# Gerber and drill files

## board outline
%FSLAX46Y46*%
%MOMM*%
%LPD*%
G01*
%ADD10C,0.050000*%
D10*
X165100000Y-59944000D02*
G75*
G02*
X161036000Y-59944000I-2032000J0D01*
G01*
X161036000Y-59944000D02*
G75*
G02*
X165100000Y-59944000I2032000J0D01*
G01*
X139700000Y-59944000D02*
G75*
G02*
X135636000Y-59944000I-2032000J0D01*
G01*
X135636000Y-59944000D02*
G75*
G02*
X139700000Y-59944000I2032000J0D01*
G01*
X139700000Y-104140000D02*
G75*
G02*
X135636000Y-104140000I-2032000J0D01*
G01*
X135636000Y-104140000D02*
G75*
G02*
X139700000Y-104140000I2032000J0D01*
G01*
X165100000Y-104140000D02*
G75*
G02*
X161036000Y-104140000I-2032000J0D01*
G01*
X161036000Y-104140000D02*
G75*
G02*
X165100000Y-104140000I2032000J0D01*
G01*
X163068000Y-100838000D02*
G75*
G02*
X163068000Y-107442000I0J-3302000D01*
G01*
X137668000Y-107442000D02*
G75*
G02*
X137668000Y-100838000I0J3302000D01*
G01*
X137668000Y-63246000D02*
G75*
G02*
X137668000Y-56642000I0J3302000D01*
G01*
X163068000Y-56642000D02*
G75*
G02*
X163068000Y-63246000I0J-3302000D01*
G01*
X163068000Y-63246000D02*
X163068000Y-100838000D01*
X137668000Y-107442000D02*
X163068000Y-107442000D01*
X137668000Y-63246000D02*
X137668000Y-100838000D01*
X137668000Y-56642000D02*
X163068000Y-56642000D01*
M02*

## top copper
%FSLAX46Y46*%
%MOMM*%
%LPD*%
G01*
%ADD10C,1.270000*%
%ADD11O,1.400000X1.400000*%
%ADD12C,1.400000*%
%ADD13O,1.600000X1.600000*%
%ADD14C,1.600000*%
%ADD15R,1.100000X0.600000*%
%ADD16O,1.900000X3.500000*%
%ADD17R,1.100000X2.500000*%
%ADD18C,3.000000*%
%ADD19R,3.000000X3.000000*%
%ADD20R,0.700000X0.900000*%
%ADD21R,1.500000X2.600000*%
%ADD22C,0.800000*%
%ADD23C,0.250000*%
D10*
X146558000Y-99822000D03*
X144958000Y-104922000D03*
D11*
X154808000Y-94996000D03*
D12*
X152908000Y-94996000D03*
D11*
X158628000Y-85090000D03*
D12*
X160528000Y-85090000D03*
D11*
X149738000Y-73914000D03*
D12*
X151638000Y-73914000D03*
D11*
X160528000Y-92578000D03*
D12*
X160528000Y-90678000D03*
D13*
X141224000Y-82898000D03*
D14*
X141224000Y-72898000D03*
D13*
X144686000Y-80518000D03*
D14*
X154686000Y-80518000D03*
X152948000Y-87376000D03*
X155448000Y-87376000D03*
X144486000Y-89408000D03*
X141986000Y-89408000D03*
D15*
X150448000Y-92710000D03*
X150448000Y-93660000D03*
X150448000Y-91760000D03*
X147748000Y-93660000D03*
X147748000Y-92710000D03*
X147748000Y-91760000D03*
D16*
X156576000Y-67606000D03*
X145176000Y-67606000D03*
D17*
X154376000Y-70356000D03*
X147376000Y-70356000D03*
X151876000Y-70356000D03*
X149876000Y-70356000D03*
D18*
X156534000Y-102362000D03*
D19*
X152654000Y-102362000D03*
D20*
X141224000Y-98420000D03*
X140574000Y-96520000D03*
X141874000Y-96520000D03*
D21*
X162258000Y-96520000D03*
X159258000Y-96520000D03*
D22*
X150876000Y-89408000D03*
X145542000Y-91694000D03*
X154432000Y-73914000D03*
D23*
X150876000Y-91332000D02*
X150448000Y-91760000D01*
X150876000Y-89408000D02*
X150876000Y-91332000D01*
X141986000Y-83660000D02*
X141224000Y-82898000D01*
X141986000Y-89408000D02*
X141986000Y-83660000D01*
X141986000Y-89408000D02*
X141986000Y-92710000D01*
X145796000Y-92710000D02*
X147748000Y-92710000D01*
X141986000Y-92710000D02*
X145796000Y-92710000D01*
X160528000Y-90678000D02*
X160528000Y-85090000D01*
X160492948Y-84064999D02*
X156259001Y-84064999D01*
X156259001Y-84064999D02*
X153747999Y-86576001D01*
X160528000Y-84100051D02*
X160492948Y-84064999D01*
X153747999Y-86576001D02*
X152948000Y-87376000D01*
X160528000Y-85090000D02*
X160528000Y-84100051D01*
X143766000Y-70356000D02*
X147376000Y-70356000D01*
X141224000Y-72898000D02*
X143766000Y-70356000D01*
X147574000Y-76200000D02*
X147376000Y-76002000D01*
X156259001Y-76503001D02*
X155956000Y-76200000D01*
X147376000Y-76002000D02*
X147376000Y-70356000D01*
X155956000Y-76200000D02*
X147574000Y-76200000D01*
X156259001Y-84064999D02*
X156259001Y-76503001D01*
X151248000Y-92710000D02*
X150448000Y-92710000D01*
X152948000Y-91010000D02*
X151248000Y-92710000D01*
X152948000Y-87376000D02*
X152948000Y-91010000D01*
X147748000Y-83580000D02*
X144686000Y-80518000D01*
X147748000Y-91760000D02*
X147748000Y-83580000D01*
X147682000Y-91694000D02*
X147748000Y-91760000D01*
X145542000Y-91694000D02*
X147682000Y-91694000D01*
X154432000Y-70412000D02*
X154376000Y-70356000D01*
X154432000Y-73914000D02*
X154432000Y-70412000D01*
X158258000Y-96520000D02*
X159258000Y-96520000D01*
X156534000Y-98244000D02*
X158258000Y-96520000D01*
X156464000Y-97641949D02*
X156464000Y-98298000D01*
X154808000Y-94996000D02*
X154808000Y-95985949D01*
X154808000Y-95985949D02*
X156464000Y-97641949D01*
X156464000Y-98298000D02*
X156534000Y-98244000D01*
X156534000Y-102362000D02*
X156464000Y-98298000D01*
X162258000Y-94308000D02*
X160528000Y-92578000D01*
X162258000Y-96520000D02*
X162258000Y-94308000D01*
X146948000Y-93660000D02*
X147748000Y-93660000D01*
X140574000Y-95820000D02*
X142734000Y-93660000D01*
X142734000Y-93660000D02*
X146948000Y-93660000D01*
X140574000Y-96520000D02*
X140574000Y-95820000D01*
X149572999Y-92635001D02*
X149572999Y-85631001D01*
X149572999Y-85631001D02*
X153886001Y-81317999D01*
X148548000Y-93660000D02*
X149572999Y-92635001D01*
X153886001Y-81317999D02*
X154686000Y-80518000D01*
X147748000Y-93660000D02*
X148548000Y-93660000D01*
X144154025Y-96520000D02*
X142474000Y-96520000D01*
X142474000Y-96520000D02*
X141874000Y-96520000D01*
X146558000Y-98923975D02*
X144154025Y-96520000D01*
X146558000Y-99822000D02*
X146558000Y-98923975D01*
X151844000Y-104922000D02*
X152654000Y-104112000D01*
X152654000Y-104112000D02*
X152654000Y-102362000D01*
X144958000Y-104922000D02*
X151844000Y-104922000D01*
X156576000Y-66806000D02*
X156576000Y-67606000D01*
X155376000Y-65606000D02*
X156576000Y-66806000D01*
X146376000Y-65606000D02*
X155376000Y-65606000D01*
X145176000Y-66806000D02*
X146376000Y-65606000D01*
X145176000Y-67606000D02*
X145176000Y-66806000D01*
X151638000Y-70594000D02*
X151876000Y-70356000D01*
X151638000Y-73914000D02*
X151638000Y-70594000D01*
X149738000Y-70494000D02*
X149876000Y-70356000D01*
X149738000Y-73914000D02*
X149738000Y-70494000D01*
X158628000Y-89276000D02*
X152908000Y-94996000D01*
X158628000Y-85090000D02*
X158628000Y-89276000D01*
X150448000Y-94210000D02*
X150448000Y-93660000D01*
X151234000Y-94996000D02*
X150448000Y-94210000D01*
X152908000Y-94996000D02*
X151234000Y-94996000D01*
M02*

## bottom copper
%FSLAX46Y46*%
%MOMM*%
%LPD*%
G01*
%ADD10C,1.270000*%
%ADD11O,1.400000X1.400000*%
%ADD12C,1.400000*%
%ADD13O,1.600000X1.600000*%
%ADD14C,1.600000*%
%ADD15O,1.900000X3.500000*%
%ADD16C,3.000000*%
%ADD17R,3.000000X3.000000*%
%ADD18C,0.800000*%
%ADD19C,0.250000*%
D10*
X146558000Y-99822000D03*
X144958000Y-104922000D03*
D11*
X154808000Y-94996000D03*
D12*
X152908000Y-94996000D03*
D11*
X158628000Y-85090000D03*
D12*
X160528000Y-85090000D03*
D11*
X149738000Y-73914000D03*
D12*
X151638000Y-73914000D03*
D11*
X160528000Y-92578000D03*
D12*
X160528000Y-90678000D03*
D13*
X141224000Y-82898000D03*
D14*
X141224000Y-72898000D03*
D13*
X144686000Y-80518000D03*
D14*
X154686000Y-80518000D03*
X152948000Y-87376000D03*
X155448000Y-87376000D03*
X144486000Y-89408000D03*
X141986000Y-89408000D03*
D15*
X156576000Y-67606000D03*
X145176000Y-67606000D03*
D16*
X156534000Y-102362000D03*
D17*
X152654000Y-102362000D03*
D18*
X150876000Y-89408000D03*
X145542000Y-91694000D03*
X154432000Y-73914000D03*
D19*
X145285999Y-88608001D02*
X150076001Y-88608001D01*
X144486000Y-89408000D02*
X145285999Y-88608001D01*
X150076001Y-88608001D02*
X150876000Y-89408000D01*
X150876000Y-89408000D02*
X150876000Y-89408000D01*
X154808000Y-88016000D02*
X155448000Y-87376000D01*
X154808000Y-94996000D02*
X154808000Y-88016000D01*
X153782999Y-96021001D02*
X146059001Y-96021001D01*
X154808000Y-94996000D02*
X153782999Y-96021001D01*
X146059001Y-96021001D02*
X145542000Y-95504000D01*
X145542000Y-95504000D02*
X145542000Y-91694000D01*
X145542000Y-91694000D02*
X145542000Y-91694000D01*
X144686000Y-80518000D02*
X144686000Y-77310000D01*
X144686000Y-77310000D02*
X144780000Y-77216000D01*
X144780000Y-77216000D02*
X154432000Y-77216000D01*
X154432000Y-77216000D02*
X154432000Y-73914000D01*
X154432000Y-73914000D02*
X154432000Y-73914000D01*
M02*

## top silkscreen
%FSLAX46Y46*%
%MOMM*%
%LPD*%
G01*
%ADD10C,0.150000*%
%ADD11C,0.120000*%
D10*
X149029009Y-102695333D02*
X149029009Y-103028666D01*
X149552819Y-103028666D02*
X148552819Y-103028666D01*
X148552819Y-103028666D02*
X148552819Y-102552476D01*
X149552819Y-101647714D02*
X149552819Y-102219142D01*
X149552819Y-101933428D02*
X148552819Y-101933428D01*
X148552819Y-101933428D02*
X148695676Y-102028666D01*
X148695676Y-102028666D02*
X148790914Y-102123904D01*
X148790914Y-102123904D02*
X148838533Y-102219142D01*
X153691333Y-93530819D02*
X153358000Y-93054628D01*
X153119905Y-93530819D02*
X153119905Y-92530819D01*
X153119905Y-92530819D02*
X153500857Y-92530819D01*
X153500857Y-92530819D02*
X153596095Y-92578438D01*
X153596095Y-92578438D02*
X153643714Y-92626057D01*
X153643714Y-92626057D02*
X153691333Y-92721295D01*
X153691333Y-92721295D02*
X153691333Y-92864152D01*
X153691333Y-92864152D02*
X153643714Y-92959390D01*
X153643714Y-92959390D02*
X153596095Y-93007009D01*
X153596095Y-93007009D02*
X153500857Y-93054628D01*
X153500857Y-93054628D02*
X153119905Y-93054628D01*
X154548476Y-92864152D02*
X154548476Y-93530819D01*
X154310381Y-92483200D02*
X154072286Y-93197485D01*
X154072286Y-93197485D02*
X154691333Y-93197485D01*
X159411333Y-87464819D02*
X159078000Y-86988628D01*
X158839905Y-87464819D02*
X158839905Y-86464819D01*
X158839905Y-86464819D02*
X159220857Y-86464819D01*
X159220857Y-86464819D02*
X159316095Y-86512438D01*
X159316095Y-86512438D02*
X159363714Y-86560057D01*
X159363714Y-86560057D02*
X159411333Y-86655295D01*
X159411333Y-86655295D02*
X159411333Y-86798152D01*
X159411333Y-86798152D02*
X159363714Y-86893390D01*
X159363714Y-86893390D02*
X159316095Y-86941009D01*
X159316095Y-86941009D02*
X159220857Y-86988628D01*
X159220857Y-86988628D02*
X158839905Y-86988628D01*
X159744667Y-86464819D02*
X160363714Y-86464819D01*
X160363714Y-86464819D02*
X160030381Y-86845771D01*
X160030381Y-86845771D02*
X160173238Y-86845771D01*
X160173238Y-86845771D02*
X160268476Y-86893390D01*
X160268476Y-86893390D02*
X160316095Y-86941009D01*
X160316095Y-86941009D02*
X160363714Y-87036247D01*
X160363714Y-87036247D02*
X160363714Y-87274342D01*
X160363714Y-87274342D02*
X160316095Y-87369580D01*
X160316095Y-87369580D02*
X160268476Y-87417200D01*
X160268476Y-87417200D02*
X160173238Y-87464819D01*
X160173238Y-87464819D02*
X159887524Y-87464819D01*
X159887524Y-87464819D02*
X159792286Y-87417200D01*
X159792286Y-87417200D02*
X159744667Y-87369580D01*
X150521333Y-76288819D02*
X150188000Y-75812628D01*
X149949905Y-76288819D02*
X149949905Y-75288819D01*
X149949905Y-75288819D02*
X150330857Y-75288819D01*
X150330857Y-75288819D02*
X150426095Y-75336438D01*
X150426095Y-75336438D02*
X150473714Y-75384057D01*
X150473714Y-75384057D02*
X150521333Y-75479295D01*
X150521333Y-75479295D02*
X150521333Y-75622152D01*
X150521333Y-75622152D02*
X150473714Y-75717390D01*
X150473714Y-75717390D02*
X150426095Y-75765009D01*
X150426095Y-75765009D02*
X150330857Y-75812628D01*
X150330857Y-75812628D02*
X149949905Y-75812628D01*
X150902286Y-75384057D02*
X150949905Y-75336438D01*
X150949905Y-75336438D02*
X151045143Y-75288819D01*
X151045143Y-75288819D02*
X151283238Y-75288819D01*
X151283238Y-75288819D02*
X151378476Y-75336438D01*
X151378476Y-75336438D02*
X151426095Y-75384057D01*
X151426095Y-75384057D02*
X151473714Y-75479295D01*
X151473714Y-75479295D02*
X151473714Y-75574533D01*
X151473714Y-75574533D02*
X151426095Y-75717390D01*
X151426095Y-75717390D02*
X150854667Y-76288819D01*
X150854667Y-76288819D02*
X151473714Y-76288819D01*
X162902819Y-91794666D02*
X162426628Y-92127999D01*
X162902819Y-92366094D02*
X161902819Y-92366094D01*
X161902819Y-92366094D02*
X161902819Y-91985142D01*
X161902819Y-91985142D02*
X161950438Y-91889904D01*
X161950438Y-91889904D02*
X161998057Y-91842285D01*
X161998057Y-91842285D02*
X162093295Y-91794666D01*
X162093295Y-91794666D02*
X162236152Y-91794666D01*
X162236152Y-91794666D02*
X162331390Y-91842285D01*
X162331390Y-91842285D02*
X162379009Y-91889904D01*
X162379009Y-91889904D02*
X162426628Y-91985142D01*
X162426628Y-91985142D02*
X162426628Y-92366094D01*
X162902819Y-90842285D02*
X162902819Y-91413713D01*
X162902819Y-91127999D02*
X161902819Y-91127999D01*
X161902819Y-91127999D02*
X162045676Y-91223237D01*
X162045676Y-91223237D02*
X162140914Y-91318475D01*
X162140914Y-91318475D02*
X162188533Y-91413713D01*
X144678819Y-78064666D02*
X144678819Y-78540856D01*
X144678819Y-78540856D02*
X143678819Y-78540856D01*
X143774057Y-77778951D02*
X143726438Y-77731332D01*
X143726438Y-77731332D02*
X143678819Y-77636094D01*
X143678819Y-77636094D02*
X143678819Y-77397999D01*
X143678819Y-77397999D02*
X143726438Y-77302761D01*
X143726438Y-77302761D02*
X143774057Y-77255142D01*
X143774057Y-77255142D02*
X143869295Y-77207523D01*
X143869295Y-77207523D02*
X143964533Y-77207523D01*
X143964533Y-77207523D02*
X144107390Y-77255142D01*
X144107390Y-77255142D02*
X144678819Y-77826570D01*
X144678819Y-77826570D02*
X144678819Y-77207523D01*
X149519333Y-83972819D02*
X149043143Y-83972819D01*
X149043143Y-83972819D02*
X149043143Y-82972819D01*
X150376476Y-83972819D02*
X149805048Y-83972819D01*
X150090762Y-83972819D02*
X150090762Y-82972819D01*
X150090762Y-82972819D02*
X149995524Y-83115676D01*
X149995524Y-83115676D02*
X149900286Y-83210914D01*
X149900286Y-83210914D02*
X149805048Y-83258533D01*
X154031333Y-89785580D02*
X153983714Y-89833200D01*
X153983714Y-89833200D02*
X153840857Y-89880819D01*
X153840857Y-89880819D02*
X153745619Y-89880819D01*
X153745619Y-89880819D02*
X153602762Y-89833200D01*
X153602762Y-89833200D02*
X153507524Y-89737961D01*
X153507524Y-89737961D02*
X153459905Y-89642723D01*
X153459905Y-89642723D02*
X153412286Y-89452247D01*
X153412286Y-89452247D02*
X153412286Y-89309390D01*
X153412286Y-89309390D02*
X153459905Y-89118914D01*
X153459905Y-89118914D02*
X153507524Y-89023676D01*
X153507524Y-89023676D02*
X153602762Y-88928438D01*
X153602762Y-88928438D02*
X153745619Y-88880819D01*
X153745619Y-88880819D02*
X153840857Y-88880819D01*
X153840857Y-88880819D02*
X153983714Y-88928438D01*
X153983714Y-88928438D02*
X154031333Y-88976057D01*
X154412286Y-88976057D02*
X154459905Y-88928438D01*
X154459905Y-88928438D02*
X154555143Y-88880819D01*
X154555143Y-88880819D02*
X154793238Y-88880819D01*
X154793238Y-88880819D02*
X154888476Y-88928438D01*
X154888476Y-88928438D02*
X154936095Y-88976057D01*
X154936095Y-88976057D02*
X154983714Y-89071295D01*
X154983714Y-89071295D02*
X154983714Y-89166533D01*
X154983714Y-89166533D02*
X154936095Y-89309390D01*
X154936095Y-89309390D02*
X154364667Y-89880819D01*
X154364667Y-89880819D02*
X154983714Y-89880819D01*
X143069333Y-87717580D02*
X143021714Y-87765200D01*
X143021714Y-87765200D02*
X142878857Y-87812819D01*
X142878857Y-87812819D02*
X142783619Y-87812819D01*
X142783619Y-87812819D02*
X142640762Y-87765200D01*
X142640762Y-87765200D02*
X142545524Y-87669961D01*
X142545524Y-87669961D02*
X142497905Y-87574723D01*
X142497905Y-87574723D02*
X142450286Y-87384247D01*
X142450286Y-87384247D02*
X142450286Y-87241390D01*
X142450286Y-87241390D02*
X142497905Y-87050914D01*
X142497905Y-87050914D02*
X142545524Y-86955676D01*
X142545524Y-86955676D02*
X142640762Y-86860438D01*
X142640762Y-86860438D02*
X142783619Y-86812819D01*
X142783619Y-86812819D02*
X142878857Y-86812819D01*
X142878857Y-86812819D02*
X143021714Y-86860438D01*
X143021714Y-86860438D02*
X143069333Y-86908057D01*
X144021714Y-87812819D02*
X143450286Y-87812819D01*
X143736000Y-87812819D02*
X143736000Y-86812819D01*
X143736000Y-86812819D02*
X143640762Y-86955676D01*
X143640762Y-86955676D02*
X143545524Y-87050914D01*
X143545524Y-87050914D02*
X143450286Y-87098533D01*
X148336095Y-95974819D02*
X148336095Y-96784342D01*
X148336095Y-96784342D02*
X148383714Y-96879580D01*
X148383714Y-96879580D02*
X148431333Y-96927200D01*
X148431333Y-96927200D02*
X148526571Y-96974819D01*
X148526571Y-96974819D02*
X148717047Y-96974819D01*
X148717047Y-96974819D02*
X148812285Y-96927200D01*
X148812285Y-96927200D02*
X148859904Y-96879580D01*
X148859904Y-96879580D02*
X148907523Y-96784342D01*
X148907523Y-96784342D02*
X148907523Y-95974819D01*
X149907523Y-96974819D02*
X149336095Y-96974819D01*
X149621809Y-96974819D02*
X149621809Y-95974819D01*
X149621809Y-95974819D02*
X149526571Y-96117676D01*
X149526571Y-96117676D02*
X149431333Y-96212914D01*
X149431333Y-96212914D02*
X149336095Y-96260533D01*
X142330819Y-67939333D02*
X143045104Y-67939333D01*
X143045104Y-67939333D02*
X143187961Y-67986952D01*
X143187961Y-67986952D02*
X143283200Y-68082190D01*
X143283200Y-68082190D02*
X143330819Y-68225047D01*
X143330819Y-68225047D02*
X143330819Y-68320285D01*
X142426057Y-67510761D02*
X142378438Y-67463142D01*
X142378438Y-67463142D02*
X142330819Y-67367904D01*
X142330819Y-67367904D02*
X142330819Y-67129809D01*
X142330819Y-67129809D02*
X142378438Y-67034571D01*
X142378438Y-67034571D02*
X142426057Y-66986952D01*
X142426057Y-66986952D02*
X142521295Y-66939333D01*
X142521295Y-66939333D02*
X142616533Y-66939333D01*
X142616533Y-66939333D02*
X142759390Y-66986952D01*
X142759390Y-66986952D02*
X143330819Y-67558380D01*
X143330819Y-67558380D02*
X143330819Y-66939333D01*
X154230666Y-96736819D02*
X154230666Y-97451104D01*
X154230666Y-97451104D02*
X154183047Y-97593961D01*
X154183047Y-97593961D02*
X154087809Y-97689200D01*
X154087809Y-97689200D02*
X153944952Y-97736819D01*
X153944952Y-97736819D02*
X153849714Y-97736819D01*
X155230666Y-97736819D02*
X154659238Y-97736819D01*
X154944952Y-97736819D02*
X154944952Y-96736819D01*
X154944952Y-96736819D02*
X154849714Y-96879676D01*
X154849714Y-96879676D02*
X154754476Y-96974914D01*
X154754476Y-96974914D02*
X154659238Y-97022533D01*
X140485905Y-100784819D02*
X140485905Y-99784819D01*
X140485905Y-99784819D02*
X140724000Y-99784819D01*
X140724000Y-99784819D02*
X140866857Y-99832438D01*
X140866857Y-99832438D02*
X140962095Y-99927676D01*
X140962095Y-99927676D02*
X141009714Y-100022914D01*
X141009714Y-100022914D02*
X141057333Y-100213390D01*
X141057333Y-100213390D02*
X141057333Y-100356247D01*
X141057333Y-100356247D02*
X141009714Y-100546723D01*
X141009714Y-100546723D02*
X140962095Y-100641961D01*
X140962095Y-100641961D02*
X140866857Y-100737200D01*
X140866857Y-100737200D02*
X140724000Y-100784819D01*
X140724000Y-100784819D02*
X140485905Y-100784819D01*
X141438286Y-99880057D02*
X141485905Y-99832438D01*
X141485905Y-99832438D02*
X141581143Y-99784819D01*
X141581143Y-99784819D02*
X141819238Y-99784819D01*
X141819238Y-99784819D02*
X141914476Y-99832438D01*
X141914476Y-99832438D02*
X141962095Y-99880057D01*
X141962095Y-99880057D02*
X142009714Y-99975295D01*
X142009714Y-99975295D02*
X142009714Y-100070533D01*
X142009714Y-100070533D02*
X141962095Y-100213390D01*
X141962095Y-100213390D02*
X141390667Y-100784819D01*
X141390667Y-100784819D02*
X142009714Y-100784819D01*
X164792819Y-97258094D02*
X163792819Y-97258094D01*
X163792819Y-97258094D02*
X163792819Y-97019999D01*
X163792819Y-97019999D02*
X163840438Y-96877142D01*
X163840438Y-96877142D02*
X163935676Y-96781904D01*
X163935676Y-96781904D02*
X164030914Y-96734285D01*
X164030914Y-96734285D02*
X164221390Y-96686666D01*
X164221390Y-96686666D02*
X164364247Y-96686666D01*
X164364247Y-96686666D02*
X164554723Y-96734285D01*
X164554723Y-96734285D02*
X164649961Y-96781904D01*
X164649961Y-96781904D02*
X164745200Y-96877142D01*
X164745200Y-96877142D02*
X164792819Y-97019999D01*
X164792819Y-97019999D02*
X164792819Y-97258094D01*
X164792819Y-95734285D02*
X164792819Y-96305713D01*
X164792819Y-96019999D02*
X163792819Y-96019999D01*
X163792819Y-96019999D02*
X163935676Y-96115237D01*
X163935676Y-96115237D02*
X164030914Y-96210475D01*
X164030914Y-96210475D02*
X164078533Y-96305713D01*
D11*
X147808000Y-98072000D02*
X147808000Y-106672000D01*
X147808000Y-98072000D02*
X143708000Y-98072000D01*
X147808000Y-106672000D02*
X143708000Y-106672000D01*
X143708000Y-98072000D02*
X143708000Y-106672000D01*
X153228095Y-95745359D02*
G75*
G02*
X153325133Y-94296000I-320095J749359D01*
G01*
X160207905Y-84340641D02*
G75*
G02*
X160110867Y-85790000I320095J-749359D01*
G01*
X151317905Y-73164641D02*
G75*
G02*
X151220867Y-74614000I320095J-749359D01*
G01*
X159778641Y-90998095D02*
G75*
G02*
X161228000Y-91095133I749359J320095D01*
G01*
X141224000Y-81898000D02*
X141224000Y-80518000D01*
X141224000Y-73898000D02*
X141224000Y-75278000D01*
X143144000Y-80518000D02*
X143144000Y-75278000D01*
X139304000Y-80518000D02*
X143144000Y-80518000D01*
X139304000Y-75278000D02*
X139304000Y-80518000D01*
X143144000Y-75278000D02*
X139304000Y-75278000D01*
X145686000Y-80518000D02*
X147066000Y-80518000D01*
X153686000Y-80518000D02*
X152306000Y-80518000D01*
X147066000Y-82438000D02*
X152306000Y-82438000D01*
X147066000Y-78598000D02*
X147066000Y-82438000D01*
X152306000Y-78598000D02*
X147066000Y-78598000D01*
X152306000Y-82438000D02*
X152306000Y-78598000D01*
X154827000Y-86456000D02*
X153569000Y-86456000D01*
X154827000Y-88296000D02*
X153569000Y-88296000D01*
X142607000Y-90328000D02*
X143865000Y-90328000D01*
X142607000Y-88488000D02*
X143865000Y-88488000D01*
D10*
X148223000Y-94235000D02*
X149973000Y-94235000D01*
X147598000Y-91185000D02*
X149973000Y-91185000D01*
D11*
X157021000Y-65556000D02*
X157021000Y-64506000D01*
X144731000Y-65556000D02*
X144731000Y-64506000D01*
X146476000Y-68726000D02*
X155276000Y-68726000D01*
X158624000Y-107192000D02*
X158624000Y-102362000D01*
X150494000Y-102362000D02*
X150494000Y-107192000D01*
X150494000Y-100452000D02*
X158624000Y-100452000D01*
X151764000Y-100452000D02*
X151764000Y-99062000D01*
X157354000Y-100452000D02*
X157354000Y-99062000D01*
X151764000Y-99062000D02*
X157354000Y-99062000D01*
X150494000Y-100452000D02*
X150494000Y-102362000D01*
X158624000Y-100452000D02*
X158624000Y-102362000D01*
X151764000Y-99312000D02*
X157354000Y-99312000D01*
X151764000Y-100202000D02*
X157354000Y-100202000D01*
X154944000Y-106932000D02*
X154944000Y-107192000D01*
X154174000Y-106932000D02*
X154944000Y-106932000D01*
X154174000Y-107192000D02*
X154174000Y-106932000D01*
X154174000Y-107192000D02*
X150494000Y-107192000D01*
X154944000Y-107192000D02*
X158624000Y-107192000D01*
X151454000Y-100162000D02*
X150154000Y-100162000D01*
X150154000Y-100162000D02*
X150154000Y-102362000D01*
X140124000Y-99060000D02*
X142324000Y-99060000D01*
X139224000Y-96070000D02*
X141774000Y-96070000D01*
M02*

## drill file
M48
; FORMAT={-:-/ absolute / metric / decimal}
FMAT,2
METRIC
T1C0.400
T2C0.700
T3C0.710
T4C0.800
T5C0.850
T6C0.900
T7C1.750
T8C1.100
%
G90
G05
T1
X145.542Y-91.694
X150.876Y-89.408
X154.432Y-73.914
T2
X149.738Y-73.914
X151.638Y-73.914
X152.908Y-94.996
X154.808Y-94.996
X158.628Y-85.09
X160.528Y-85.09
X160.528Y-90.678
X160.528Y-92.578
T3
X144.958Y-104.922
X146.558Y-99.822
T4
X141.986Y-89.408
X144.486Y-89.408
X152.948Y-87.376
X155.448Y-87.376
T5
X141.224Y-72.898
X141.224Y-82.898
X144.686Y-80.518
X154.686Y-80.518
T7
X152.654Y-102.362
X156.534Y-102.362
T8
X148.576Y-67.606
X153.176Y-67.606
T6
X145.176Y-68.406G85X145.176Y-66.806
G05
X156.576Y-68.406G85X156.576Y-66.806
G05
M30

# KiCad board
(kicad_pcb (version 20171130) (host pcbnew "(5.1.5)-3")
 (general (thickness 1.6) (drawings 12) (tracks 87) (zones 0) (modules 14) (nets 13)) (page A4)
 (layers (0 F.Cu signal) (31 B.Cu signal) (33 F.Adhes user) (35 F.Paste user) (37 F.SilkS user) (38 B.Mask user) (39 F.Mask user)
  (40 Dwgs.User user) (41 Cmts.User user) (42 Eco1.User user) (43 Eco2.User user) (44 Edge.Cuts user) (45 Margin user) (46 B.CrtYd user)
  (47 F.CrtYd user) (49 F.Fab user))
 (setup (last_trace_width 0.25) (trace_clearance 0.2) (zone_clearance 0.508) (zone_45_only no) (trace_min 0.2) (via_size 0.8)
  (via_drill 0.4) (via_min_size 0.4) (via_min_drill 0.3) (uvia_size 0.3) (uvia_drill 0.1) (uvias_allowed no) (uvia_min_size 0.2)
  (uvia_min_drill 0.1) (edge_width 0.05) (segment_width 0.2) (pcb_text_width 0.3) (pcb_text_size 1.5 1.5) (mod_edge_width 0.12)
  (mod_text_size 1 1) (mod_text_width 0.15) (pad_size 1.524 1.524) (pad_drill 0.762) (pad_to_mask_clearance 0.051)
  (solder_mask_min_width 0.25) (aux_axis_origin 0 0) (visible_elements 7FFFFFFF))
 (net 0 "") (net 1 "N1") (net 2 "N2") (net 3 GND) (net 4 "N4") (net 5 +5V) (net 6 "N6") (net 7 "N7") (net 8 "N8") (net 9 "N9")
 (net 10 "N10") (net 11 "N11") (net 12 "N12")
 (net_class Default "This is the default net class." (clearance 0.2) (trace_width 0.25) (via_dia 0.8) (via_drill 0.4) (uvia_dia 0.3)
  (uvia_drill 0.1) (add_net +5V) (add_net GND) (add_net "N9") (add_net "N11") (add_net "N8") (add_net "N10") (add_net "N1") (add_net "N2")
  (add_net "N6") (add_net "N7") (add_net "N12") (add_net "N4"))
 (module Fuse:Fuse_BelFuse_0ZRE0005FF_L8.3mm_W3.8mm (layer F.Cu) (at 146.558 99.822 270)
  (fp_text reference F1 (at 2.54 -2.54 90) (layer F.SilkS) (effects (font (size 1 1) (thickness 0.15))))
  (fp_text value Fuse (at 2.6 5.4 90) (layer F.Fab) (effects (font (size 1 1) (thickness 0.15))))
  (fp_line (start -1.75 -1.25) (end 6.85 -1.25) (layer F.SilkS) (width 0.12))
  (fp_line (start -1.75 -1.25) (end -1.75 2.85) (layer F.SilkS) (width 0.12))
  (fp_line (start 6.85 -1.25) (end 6.85 2.85) (layer F.SilkS) (width 0.12))
  (fp_line (start -1.75 2.85) (end 6.85 2.85) (layer F.SilkS) (width 0.12))
  (pad 1 thru_hole circle (at 0 0 270) (size 1.27 1.27) (drill 0.71) (layers *.Cu *.Mask) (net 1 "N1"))
  (pad 2 thru_hole circle (at 5.1 1.6 270) (size 1.27 1.27) (drill 0.71) (layers *.Cu *.Mask) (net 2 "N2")))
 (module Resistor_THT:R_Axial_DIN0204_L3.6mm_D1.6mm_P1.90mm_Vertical (layer F.Cu) (at 152.908 94.996)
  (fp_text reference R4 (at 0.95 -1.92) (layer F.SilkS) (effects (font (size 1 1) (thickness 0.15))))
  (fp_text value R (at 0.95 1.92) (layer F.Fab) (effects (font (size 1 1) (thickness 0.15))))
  (fp_arc (start 0 0) (end 0.417133 -0.7) (angle -233.92106) (layer F.SilkS) (width 0.12))
  (pad 2 thru_hole oval (at 1.9 0) (size 1.4 1.4) (drill 0.7) (layers *.Cu *.Mask) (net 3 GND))
  (pad 1 thru_hole circle (at 0 0) (size 1.4 1.4) (drill 0.7) (layers *.Cu *.Mask) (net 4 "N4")))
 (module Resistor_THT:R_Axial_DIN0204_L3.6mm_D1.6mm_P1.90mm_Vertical (layer F.Cu) (at 160.528 85.09 180)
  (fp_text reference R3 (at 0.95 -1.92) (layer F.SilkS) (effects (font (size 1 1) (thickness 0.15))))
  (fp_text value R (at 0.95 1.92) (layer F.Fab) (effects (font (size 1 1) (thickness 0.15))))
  (fp_arc (start 0 0) (end 0.417133 -0.7) (angle -233.92106) (layer F.SilkS) (width 0.12))
  (pad 2 thru_hole oval (at 1.9 0 180) (size 1.4 1.4) (drill 0.7) (layers *.Cu *.Mask) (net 4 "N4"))
  (pad 1 thru_hole circle (at 0 0 180) (size 1.4 1.4) (drill 0.7) (layers *.Cu *.Mask) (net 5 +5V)))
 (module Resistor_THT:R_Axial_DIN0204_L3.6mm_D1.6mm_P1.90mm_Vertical (layer F.Cu) (at 151.638 73.914 180)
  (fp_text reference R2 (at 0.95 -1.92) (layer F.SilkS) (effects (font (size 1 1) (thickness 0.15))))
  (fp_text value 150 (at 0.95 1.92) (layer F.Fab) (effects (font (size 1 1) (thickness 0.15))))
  (fp_arc (start 0 0) (end 0.417133 -0.7) (angle -233.92106) (layer F.SilkS) (width 0.12))
  (pad 2 thru_hole oval (at 1.9 0 180) (size 1.4 1.4) (drill 0.7) (layers *.Cu *.Mask) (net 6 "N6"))
  (pad 1 thru_hole circle (at 0 0 180) (size 1.4 1.4) (drill 0.7) (layers *.Cu *.Mask) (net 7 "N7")))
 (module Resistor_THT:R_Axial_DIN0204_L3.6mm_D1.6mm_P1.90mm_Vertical (layer F.Cu) (at 160.528 90.678 270)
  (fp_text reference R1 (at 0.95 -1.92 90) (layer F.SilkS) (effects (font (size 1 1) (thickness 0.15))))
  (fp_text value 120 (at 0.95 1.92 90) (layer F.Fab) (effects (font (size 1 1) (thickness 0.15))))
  (fp_arc (start 0 0) (end 0.417133 -0.7) (angle -233.92106) (layer F.SilkS) (width 0.12))
  (pad 2 thru_hole oval (at 1.9 0 270) (size 1.4 1.4) (drill 0.7) (layers *.Cu *.Mask) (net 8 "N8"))
  (pad 1 thru_hole circle (at 0 0 270) (size 1.4 1.4) (drill 0.7) (layers *.Cu *.Mask) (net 5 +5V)))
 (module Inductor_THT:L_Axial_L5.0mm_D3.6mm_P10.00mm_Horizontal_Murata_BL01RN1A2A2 (layer F.Cu) (at 141.224 72.898 270)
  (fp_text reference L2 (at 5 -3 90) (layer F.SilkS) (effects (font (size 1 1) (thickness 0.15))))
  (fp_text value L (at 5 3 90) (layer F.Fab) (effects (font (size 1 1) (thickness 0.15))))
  (fp_line (start 9 0) (end 7.62 0) (layer F.SilkS) (width 0.12))
  (fp_line (start 1 0) (end 2.38 0) (layer F.SilkS) (width 0.12))
  (fp_line (start 7.62 -1.92) (end 2.38 -1.92) (layer F.SilkS) (width 0.12))
  (fp_line (start 7.62 1.92) (end 7.62 -1.92) (layer F.SilkS) (width 0.12))
  (fp_line (start 2.38 1.92) (end 7.62 1.92) (layer F.SilkS) (width 0.12))
  (fp_line (start 2.38 -1.92) (end 2.38 1.92) (layer F.SilkS) (width 0.12))
  (pad 2 thru_hole oval (at 10 0 270) (size 1.6 1.6) (drill 0.85) (layers *.Cu *.Mask) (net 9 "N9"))
  (pad 1 thru_hole circle (at 0 0 270) (size 1.6 1.6) (drill 0.85) (layers *.Cu *.Mask) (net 5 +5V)))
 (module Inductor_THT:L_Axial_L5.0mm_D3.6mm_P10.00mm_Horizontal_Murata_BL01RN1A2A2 (layer F.Cu) (at 154.686 80.518 180)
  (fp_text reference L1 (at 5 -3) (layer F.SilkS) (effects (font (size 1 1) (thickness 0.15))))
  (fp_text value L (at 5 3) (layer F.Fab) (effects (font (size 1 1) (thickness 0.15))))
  (fp_line (start 9 0) (end 7.62 0) (layer F.SilkS) (width 0.12))
  (fp_line (start 1 0) (end 2.38 0) (layer F.SilkS) (width 0.12))
  (fp_line (start 7.62 -1.92) (end 2.38 -1.92) (layer F.SilkS) (width 0.12))
  (fp_line (start 7.62 1.92) (end 7.62 -1.92) (layer F.SilkS) (width 0.12))
  (fp_line (start 2.38 1.92) (end 7.62 1.92) (layer F.SilkS) (width 0.12))
  (fp_line (start 2.38 -1.92) (end 2.38 1.92) (layer F.SilkS) (width 0.12))
  (pad 2 thru_hole oval (at 10 0 180) (size 1.6 1.6) (drill 0.85) (layers *.Cu *.Mask) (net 3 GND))
  (pad 1 thru_hole circle (at 0 0 180) (size 1.6 1.6) (drill 0.85) (layers *.Cu *.Mask) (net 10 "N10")))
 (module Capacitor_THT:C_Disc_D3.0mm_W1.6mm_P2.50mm (layer F.Cu) (at 155.448 87.376 180)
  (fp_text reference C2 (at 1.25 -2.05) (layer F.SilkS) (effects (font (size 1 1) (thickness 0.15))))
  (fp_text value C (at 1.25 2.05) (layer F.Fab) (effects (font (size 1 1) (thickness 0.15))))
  (fp_line (start 0.621 0.92) (end 1.879 0.92) (layer F.SilkS) (width 0.12))
  (fp_line (start 0.621 -0.92) (end 1.879 -0.92) (layer F.SilkS) (width 0.12))
  (pad 2 thru_hole circle (at 2.5 0 180) (size 1.6 1.6) (drill 0.8) (layers *.Cu *.Mask) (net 5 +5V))
  (pad 1 thru_hole circle (at 0 0 180) (size 1.6 1.6) (drill 0.8) (layers *.Cu *.Mask) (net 3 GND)))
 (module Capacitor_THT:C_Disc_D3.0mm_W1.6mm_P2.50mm (layer F.Cu) (at 141.986 89.408)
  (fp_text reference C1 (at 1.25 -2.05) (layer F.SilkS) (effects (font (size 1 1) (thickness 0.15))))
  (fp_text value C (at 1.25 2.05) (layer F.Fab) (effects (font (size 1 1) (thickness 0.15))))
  (fp_line (start 0.621 0.92) (end 1.879 0.92) (layer F.SilkS) (width 0.12))
  (fp_line (start 0.621 -0.92) (end 1.879 -0.92) (layer F.SilkS) (width 0.12))
  (pad 2 thru_hole circle (at 2.5 0) (size 1.6 1.6) (drill 0.8) (layers *.Cu *.Mask) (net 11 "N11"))
  (pad 1 thru_hole circle (at 0 0) (size 1.6 1.6) (drill 0.8) (layers *.Cu *.Mask) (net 9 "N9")))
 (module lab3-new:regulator (layer F.Cu) (at 149.098 92.71)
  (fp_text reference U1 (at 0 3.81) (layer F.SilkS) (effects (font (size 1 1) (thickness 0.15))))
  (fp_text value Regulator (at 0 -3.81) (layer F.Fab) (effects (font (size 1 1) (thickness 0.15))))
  (fp_line (start -0.875 1.525) (end 0.875 1.525) (layer F.SilkS) (width 0.15))
  (fp_line (start -1.5 -1.525) (end 0.875 -1.525) (layer F.SilkS) (width 0.15))
  (pad 5 smd rect (at 1.35 0) (size 1.1 0.6) (layers F.Cu F.Paste F.Mask) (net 5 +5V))
  (pad 4 smd rect (at 1.35 0.95) (size 1.1 0.6) (layers F.Cu F.Paste F.Mask) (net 4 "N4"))
  (pad 6 smd rect (at 1.35 -0.95) (size 1.1 0.6) (layers F.Cu F.Paste F.Mask) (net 11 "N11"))
  (pad 3 smd rect (at -1.35 0.95) (size 1.1 0.6) (layers F.Cu F.Paste F.Mask) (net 10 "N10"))
  (pad 2 smd rect (at -1.35 0) (size 1.1 0.6) (layers F.Cu F.Paste F.Mask) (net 9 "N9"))
  (pad 1 smd rect (at -1.35 -0.95) (size 1.1 0.6) (layers F.Cu F.Paste F.Mask) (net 3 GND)))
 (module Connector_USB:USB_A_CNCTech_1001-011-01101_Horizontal (layer F.Cu) (at 150.876 60.706 90)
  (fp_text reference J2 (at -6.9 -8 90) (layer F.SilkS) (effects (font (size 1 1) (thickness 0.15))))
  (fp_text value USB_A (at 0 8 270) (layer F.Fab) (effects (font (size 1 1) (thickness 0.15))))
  (fp_line (start -4.85 6.145) (end -3.8 6.145) (layer F.SilkS) (width 0.12))
  (fp_line (start -4.85 -6.145) (end -3.8 -6.145) (layer F.SilkS) (width 0.12))
  (fp_line (start -8.02 -4.4) (end -8.02 4.4) (layer F.SilkS) (width 0.12))
  (pad "" np_thru_hole circle (at -6.9 2.3 90) (size 1.1 1.1) (drill 1.1) (layers *.Cu *.Mask))
  (pad "" np_thru_hole circle (at -6.9 -2.3 90) (size 1.1 1.1) (drill 1.1) (layers *.Cu *.Mask))
  (pad 5 thru_hole oval (at -6.9 5.7 90) (size 3.5 1.9) (drill oval 2.5 0.9) (layers *.Cu *.Mask) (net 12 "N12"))
  (pad 5 thru_hole oval (at -6.9 -5.7 90) (size 3.5 1.9) (drill oval 2.5 0.9) (layers *.Cu *.Mask) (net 12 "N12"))
  (pad 4 smd rect (at -9.65 3.5 90) (size 2.5 1.1) (layers F.Cu F.Paste F.Mask) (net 3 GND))
  (pad 1 smd rect (at -9.65 -3.5 90) (size 2.5 1.1) (layers F.Cu F.Paste F.Mask) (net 5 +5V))
  (pad 3 smd rect (at -9.65 1 90) (size 2.5 1.1) (layers F.Cu F.Paste F.Mask) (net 7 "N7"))
  (pad 2 smd rect (at -9.65 -1 90) (size 2.5 1.1) (layers F.Cu F.Paste F.Mask) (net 6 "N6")))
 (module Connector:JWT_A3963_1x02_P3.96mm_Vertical (layer F.Cu) (at 152.654 102.362)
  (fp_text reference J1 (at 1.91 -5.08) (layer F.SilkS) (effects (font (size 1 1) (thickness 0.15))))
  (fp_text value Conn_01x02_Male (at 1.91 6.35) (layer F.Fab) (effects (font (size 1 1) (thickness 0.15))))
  (fp_line (start 5.97 4.83) (end 5.97 0) (layer F.SilkS) (width 0.12))
  (fp_line (start -2.16 0) (end -2.16 4.83) (layer F.SilkS) (width 0.12))
  (fp_line (start -2.16 -1.91) (end 5.97 -1.91) (layer F.SilkS) (width 0.12))
  (fp_line (start -0.89 -1.91) (end -0.89 -3.3) (layer F.SilkS) (width 0.12))
  (fp_line (start 4.7 -1.91) (end 4.7 -3.3) (layer F.SilkS) (width 0.12))
  (fp_line (start -0.89 -3.3) (end 4.7 -3.3) (layer F.SilkS) (width 0.12))
  (fp_line (start -2.16 -1.91) (end -2.16 0) (layer F.SilkS) (width 0.12))
  (fp_line (start 5.97 -1.91) (end 5.97 0) (layer F.SilkS) (width 0.12))
  (fp_line (start -0.89 -3.05) (end 4.7 -3.05) (layer F.SilkS) (width 0.12))
  (fp_line (start -0.89 -2.16) (end 4.7 -2.16) (layer F.SilkS) (width 0.12))
  (fp_line (start 2.29 4.57) (end 2.29 4.83) (layer F.SilkS) (width 0.12))
  (fp_line (start 1.52 4.57) (end 2.29 4.57) (layer F.SilkS) (width 0.12))
  (fp_line (start 1.52 4.83) (end 1.52 4.57) (layer F.SilkS) (width 0.12))
  (fp_line (start 1.52 4.83) (end -2.16 4.83) (layer F.SilkS) (width 0.12))
  (fp_line (start 2.29 4.83) (end 5.97 4.83) (layer F.SilkS) (width 0.12))
  (fp_line (start -1.2 -2.2) (end -2.5 -2.2) (layer F.SilkS) (width 0.12))
  (fp_line (start -2.5 -2.2) (end -2.5 0) (layer F.SilkS) (width 0.12))
  (pad 2 thru_hole circle (at 3.88 0) (size 3 3) (drill 1.75) (layers *.Cu *.Mask) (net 3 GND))
  (pad 1 thru_hole rect (at 0 0) (size 3 3) (drill 1.75) (layers *.Cu *.Mask) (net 2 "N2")))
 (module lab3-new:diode (layer F.Cu) (at 141.224 96.52)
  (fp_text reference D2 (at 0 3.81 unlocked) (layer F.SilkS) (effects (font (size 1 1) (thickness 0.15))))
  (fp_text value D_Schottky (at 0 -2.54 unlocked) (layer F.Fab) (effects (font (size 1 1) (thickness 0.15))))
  (fp_line (start -1.1 2.54) (end 1.1 2.54) (layer F.SilkS) (width 0.12))
  (fp_line (start -2 -0.45) (end 0.55 -0.45) (layer F.SilkS) (width 0.12))
  (pad 3 smd rect (at 0 1.9) (size 0.7 0.9) (layers F.Cu F.Paste F.Mask))
  (pad 1 smd rect (at -0.65 0) (size 0.7 0.9) (layers F.Cu F.Paste F.Mask) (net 10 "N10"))
  (pad 2 smd rect (at 0.65 0) (size 0.7 0.9) (layers F.Cu F.Paste F.Mask) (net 1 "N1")))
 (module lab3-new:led (layer F.Cu) (at 159.258 96.52 90)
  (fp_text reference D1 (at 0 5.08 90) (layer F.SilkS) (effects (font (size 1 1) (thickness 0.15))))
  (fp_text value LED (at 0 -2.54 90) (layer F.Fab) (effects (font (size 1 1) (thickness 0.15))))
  (pad 2 smd rect (at 0 3 90) (size 2.6 1.5) (layers F.Cu F.Paste F.Mask) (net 8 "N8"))
  (pad 1 smd rect (at 0 0 90) (size 2.6 1.5) (layers F.Cu F.Paste F.Mask) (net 3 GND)))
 (gr_circle (center 163.068 59.944) (end 163.068 61.976) (layer Edge.Cuts) (width 0.05))
 (gr_circle (center 137.668 59.944) (end 137.668 61.976) (layer Edge.Cuts) (width 0.05))
 (gr_circle (center 137.668 104.14) (end 137.668 106.172) (layer Edge.Cuts) (width 0.05))
 (gr_circle (center 163.068 104.14) (end 163.068 106.172) (layer Edge.Cuts) (width 0.05))
 (gr_arc (start 163.068 104.14) (end 163.068 107.442) (angle -180) (layer Edge.Cuts) (width 0.05))
 (gr_arc (start 137.668 104.14) (end 137.668 100.838) (angle -180) (layer Edge.Cuts) (width 0.05))
 (gr_arc (start 137.668 59.944) (end 137.668 56.642) (angle -180) (layer Edge.Cuts) (width 0.05))
 (gr_arc (start 163.068 59.944) (end 163.068 63.246) (angle -180) (layer Edge.Cuts) (width 0.05))
 (gr_line (start 163.068 63.246) (end 163.068 100.838) (layer Edge.Cuts) (width 0.05))
 (gr_line (start 137.668 107.442) (end 163.068 107.442) (layer Edge.Cuts) (width 0.05))
 (gr_line (start 137.668 63.246) (end 137.668 100.838) (layer Edge.Cuts) (width 0.05))
 (gr_line (start 137.668 56.642) (end 163.068 56.642) (layer Edge.Cuts) (width 0.05))
 (segment (start 145.285999 88.608001) (end 150.076001 88.608001) (width 0.25) (layer B.Cu) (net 11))
 (segment (start 144.486 89.408) (end 145.285999 88.608001) (width 0.25) (layer B.Cu) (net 11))
 (segment (start 150.076001 88.608001) (end 150.876 89.408) (width 0.25) (layer B.Cu) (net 11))
 (segment (start 150.876 89.408) (end 150.876 89.408) (width 0.25) (layer B.Cu) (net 11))
 (via (at 150.876 89.408) (size 0.8) (drill 0.4) (layers F.Cu B.Cu) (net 11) (status 1000000))
 (segment (start 150.876 91.332) (end 150.448 91.76) (width 0.25) (layer F.Cu) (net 11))
 (segment (start 150.876 89.408) (end 150.876 91.332) (width 0.25) (layer F.Cu) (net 11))
 (segment (start 141.986 83.66) (end 141.224 82.898) (width 0.25) (layer F.Cu) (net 9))
 (segment (start 141.986 89.408) (end 141.986 83.66) (width 0.25) (layer F.Cu) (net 9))
 (segment (start 141.986 89.408) (end 141.986 92.71) (width 0.25) (layer F.Cu) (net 9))
 (segment (start 145.796 92.71) (end 147.748 92.71) (width 0.25) (layer F.Cu) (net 9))
 (segment (start 141.986 92.71) (end 145.796 92.71) (width 0.25) (layer F.Cu) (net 9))
 (segment (start 160.528 90.678) (end 160.528 85.09) (width 0.25) (layer F.Cu) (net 5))
 (segment (start 160.492948 84.064999) (end 156.259001 84.064999) (width 0.25) (layer F.Cu) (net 5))
 (segment (start 156.259001 84.064999) (end 153.747999 86.576001) (width 0.25) (layer F.Cu) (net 5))
 (segment (start 160.528 84.100051) (end 160.492948 84.064999) (width 0.25) (layer F.Cu) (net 5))
 (segment (start 153.747999 86.576001) (end 152.948 87.376) (width 0.25) (layer F.Cu) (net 5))
 (segment (start 160.528 85.09) (end 160.528 84.100051) (width 0.25) (layer F.Cu) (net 5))
 (segment (start 143.766 70.356) (end 147.376 70.356) (width 0.25) (layer F.Cu) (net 5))
 (segment (start 141.224 72.898) (end 143.766 70.356) (width 0.25) (layer F.Cu) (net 5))
 (segment (start 147.574 76.2) (end 147.376 76.002) (width 0.25) (layer F.Cu) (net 5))
 (segment (start 156.259001 76.503001) (end 155.956 76.2) (width 0.25) (layer F.Cu) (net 5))
 (segment (start 147.376 76.002) (end 147.376 70.356) (width 0.25) (layer F.Cu) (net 5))
 (segment (start 155.956 76.2) (end 147.574 76.2) (width 0.25) (layer F.Cu) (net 5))
 (segment (start 156.259001 84.064999) (end 156.259001 76.503001) (width 0.25) (layer F.Cu) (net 5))
 (segment (start 151.248 92.71) (end 150.448 92.71) (width 0.25) (layer F.Cu) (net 5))
 (segment (start 152.948 91.01) (end 151.248 92.71) (width 0.25) (layer F.Cu) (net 5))
 (segment (start 152.948 87.376) (end 152.948 91.01) (width 0.25) (layer F.Cu) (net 5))
 (segment (start 154.808 88.016) (end 155.448 87.376) (width 0.25) (layer B.Cu) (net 3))
 (segment (start 154.808 94.996) (end 154.808 88.016) (width 0.25) (layer B.Cu) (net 3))
 (segment (start 147.748 83.58) (end 144.686 80.518) (width 0.25) (layer F.Cu) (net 3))
 (segment (start 147.748 91.76) (end 147.748 83.58) (width 0.25) (layer F.Cu) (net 3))
 (segment (start 153.782999 96.021001) (end 146.059001 96.021001) (width 0.25) (layer B.Cu) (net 3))
 (segment (start 154.808 94.996) (end 153.782999 96.021001) (width 0.25) (layer B.Cu) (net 3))
 (segment (start 146.059001 96.021001) (end 145.542 95.504) (width 0.25) (layer B.Cu) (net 3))
 (segment (start 145.542 95.504) (end 145.542 91.694) (width 0.25) (layer B.Cu) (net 3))
 (segment (start 145.542 91.694) (end 145.542 91.694) (width 0.25) (layer B.Cu) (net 3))
 (via (at 145.542 91.694) (size 0.8) (drill 0.4) (layers F.Cu B.Cu) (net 3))
 (segment (start 147.682 91.694) (end 147.748 91.76) (width 0.25) (layer F.Cu) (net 3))
 (segment (start 145.542 91.694) (end 147.682 91.694) (width 0.25) (layer F.Cu) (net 3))
 (segment (start 144.686 80.518) (end 144.686 77.31) (width 0.25) (layer B.Cu) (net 3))
 (segment (start 144.686 77.31) (end 144.78 77.216) (width 0.25) (layer B.Cu) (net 3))
 (segment (start 144.78 77.216) (end 154.432 77.216) (width 0.25) (layer B.Cu) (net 3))
 (segment (start 154.432 77.216) (end 154.432 73.914) (width 0.25) (layer B.Cu) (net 3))
 (segment (start 154.432 73.914) (end 154.432 73.914) (width 0.25) (layer B.Cu) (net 3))
 (via (at 154.432 73.914) (size 0.8) (drill 0.4) (layers F.Cu B.Cu) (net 3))
 (segment (start 154.432 70.412) (end 154.376 70.356) (width 0.25) (layer F.Cu) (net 3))
 (segment (start 154.432 73.914) (end 154.432 70.412) (width 0.25) (layer F.Cu) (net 3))
 (segment (start 158.258 96.52) (end 159.258 96.52) (width 0.25) (layer F.Cu) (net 3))
 (segment (start 156.534 98.244) (end 158.258 96.52) (width 0.25) (layer F.Cu) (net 3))
 (segment (start 156.464 97.641949) (end 156.464 98.298) (width 0.25) (layer F.Cu) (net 3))
 (segment (start 154.808 94.996) (end 154.808 95.985949) (width 0.25) (layer F.Cu) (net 3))
 (segment (start 154.808 95.985949) (end 156.464 97.641949) (width 0.25) (layer F.Cu) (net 3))
 (segment (start 156.464 98.298) (end 156.534 98.244) (width 0.25) (layer F.Cu) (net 3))
 (segment (start 156.534 102.362) (end 156.464 98.298) (width 0.25) (layer F.Cu) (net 3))
 (segment (start 162.258 94.308) (end 160.528 92.578) (width 0.25) (layer F.Cu) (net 8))
 (segment (start 162.258 96.52) (end 162.258 94.308) (width 0.25) (layer F.Cu) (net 8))
 (segment (start 146.948 93.66) (end 147.748 93.66) (width 0.25) (layer F.Cu) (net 10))
 (segment (start 140.574 95.82) (end 142.734 93.66) (width 0.25) (layer F.Cu) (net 10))
 (segment (start 142.734 93.66) (end 146.948 93.66) (width 0.25) (layer F.Cu) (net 10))
 (segment (start 140.574 96.52) (end 140.574 95.82) (width 0.25) (layer F.Cu) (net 10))
 (segment (start 149.572999 92.635001) (end 149.572999 85.631001) (width 0.25) (layer F.Cu) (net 10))
 (segment (start 149.572999 85.631001) (end 153.886001 81.317999) (width 0.25) (layer F.Cu) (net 10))
 (segment (start 148.548 93.66) (end 149.572999 92.635001) (width 0.25) (layer F.Cu) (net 10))
 (segment (start 153.886001 81.317999) (end 154.686 80.518) (width 0.25) (layer F.Cu) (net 10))
 (segment (start 147.748 93.66) (end 148.548 93.66) (width 0.25) (layer F.Cu) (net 10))
 (segment (start 144.154025 96.52) (end 142.474 96.52) (width 0.25) (layer F.Cu) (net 1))
 (segment (start 142.474 96.52) (end 141.874 96.52) (width 0.25) (layer F.Cu) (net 1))
 (segment (start 146.558 98.923975) (end 144.154025 96.52) (width 0.25) (layer F.Cu) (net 1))
 (segment (start 146.558 99.822) (end 146.558 98.923975) (width 0.25) (layer F.Cu) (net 1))
 (segment (start 151.844 104.922) (end 152.654 104.112) (width 0.25) (layer F.Cu) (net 2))
 (segment (start 152.654 104.112) (end 152.654 102.362) (width 0.25) (layer F.Cu) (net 2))
 (segment (start 144.958 104.922) (end 151.844 104.922) (width 0.25) (layer F.Cu) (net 2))
 (segment (start 156.576 66.806) (end 156.576 67.606) (width 0.25) (layer F.Cu) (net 12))
 (segment (start 155.376 65.606) (end 156.576 66.806) (width 0.25) (layer F.Cu) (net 12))
 (segment (start 146.376 65.606) (end 155.376 65.606) (width 0.25) (layer F.Cu) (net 12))
 (segment (start 145.176 66.806) (end 146.376 65.606) (width 0.25) (layer F.Cu) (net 12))
 (segment (start 145.176 67.606) (end 145.176 66.806) (width 0.25) (layer F.Cu) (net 12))
 (segment (start 151.638 70.594) (end 151.876 70.356) (width 0.25) (layer F.Cu) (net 7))
 (segment (start 151.638 73.914) (end 151.638 70.594) (width 0.25) (layer F.Cu) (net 7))
 (segment (start 149.738 70.494) (end 149.876 70.356) (width 0.25) (layer F.Cu) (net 6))
 (segment (start 149.738 73.914) (end 149.738 70.494) (width 0.25) (layer F.Cu) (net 6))
 (segment (start 158.628 89.276) (end 152.908 94.996) (width 0.25) (layer F.Cu) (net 4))
 (segment (start 158.628 85.09) (end 158.628 89.276) (width 0.25) (layer F.Cu) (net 4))
 (segment (start 150.448 94.21) (end 150.448 93.66) (width 0.25) (layer F.Cu) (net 4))
 (segment (start 151.234 94.996) (end 150.448 94.21) (width 0.25) (layer F.Cu) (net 4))
 (segment (start 152.908 94.996) (end 151.234 94.996) (width 0.25) (layer F.Cu) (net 4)))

